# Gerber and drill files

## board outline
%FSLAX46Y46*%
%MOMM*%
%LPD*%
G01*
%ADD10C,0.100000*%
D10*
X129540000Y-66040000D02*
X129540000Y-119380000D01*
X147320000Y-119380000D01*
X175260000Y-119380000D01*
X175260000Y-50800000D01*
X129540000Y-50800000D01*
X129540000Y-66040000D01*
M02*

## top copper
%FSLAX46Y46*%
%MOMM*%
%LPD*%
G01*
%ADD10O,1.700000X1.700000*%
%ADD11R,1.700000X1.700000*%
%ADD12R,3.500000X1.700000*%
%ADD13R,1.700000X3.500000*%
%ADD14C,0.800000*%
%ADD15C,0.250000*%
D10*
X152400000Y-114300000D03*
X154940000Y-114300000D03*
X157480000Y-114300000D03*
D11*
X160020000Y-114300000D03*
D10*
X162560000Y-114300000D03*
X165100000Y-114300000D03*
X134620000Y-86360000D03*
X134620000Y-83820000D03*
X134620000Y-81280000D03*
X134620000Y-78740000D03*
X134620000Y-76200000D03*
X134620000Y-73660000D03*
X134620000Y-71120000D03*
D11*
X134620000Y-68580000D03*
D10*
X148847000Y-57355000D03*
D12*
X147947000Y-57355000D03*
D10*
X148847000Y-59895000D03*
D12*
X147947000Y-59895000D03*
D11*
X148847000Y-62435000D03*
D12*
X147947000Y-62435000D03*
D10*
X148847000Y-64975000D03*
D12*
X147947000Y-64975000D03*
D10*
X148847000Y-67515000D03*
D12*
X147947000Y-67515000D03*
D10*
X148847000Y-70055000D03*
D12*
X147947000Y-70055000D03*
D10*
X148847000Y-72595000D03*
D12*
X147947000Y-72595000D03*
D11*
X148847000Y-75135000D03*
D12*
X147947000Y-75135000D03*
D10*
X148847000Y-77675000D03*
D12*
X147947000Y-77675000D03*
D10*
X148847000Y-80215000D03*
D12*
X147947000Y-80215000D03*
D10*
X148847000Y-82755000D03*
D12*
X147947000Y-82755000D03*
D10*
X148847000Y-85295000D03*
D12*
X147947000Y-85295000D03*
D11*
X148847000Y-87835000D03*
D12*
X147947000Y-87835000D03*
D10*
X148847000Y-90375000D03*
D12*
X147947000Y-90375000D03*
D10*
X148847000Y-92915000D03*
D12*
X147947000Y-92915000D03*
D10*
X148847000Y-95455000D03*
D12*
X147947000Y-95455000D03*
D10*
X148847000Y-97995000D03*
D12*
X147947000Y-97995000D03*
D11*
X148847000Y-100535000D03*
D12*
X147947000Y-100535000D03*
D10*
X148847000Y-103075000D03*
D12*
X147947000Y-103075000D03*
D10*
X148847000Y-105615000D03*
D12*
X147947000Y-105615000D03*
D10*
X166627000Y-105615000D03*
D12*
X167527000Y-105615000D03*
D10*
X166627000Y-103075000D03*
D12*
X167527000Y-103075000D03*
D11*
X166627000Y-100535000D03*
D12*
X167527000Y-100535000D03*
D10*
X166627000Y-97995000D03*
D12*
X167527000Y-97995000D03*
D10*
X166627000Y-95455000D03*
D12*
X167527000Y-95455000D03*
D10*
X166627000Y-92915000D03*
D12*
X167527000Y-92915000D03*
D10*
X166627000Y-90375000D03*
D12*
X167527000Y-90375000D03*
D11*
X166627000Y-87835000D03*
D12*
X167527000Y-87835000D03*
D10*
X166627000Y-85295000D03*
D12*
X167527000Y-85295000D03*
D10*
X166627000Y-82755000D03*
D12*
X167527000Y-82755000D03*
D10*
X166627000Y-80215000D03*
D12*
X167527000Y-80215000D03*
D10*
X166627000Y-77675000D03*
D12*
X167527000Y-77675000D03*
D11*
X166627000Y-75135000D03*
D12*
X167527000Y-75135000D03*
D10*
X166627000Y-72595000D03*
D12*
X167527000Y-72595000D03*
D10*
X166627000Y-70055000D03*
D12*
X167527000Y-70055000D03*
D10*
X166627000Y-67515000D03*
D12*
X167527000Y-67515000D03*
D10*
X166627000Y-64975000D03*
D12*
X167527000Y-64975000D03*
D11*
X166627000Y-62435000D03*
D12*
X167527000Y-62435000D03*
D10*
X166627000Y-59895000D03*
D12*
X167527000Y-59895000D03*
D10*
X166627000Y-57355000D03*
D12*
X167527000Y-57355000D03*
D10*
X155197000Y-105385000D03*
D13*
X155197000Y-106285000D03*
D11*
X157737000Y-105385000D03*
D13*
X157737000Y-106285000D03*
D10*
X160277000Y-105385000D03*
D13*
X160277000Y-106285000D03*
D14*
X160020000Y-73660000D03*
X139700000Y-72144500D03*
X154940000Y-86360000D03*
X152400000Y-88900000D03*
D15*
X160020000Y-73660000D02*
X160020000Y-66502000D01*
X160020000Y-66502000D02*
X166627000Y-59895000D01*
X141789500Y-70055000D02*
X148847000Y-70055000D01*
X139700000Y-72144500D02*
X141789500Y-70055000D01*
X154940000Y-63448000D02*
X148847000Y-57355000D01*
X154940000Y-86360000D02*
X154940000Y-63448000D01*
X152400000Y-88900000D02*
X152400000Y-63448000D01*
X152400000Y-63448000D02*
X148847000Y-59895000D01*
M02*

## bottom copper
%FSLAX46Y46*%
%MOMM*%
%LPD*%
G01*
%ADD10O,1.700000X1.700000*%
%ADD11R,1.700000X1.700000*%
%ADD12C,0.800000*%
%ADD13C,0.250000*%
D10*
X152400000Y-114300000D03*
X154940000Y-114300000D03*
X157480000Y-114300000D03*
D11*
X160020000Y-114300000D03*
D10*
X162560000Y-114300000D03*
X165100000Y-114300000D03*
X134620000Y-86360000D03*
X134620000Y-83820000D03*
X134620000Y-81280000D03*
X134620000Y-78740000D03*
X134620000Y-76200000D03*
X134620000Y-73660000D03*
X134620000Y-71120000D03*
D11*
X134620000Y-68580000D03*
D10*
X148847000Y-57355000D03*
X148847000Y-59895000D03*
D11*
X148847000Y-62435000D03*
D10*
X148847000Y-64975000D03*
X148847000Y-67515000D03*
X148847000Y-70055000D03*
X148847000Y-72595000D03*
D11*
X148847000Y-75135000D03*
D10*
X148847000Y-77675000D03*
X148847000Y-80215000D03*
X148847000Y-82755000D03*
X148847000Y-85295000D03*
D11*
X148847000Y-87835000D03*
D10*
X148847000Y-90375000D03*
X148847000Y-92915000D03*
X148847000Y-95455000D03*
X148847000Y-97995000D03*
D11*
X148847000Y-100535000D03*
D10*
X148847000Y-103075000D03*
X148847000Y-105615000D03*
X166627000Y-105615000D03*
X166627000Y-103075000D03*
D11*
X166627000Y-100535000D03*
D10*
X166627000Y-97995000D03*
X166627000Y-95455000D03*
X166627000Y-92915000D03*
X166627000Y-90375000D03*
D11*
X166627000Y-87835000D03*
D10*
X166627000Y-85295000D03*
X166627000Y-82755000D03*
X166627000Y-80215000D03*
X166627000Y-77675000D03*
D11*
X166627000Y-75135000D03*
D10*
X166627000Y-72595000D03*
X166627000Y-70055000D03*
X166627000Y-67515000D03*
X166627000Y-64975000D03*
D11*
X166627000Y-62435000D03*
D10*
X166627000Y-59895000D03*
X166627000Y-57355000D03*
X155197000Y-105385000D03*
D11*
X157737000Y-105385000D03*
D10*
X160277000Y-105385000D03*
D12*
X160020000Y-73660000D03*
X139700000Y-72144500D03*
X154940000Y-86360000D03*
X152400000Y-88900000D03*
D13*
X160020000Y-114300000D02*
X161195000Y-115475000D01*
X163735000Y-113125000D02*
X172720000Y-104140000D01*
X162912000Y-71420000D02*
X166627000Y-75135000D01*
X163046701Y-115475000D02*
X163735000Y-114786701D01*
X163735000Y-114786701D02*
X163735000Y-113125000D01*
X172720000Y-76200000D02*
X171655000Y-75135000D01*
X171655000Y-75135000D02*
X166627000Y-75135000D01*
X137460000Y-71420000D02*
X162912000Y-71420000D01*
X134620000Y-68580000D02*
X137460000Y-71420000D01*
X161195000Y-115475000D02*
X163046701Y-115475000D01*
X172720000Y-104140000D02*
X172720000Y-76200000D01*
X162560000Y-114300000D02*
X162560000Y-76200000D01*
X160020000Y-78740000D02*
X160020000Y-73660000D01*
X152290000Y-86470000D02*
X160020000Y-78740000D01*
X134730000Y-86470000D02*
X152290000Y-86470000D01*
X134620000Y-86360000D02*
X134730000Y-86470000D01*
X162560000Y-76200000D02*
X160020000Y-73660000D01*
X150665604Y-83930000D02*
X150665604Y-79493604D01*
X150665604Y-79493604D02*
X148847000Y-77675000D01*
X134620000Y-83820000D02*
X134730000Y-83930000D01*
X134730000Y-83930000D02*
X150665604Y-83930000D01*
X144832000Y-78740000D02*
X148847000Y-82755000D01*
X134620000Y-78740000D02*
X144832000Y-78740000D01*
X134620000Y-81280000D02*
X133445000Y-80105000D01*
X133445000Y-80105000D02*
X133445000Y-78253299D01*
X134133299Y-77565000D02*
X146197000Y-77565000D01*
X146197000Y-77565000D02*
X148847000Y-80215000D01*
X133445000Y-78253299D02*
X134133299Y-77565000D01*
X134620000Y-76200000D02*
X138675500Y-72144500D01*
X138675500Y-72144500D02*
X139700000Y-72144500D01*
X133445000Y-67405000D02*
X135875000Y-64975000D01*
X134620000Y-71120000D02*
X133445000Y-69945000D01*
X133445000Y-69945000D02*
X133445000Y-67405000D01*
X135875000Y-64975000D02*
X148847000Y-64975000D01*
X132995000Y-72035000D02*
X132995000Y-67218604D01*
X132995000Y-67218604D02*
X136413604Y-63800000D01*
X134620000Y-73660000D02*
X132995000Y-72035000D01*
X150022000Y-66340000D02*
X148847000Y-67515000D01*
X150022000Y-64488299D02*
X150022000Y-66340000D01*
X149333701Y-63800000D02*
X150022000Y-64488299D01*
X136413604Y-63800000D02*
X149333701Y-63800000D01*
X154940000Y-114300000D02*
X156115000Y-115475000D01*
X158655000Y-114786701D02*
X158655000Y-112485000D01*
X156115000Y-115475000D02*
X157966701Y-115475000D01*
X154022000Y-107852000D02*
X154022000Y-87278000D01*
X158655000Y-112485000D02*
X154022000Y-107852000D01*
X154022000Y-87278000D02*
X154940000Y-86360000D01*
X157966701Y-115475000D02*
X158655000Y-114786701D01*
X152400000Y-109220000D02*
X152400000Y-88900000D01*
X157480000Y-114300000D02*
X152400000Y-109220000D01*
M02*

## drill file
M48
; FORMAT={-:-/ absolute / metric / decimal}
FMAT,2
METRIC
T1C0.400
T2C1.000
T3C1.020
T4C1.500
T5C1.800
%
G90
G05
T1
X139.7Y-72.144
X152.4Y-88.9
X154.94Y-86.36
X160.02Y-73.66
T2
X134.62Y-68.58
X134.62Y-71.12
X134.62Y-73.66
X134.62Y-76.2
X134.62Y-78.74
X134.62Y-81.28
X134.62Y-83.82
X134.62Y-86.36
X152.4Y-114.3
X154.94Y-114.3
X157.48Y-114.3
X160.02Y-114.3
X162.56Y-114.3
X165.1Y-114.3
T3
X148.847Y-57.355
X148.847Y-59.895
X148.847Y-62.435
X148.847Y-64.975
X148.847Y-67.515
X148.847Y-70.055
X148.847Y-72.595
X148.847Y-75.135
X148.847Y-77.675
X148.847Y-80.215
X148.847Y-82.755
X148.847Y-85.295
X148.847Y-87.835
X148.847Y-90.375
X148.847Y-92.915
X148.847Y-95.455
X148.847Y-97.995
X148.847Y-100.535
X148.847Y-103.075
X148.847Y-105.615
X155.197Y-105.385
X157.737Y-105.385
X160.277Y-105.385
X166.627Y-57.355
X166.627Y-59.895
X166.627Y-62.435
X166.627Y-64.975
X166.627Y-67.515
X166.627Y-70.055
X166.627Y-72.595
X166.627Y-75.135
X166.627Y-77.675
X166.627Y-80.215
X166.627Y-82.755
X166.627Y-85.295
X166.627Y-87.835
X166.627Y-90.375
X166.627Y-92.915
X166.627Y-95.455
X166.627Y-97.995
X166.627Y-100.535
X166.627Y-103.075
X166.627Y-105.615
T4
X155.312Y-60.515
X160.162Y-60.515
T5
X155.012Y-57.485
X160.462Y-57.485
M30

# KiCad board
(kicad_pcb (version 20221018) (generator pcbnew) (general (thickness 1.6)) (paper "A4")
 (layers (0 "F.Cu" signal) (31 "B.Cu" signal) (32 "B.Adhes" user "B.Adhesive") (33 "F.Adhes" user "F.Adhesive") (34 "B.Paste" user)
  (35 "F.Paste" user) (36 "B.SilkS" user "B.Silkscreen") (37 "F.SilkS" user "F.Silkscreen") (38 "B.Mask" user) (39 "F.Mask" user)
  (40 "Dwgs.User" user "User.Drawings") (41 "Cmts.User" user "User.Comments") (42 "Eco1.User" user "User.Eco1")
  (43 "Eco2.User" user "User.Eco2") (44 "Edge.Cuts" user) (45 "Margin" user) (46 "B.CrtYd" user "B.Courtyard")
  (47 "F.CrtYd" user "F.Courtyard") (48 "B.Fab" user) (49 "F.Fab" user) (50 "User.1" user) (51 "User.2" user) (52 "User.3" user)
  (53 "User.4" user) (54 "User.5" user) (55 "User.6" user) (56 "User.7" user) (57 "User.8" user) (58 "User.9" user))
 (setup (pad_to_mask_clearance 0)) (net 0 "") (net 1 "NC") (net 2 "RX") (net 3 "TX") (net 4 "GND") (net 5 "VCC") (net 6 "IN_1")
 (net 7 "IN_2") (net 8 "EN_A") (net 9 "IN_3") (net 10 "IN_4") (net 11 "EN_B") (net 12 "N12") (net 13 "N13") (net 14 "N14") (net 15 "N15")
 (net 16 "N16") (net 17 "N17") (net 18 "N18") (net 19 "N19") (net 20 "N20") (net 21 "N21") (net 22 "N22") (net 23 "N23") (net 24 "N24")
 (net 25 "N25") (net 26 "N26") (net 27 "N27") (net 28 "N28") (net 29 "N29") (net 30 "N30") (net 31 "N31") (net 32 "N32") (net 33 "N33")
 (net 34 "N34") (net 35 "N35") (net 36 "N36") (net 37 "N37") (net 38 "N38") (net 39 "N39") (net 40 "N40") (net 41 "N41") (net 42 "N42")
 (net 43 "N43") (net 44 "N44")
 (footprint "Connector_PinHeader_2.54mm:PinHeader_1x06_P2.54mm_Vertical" (layer "F.Cu") (at 152.4 114.3 90)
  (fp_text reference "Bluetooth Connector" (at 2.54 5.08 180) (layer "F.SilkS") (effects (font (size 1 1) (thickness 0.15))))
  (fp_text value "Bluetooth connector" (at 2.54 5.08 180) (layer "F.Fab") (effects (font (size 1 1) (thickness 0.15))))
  (pad "1" thru_hole oval (at 0 0 90) (size 1.7 1.7) (drill 1) (layers "*.Cu" "*.Mask") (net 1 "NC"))
  (pad "2" thru_hole oval (at 0 2.54 90) (size 1.7 1.7) (drill 1) (layers "*.Cu" "*.Mask") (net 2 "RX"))
  (pad "3" thru_hole oval (at 0 5.08 90) (size 1.7 1.7) (drill 1) (layers "*.Cu" "*.Mask") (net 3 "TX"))
  (pad "4" thru_hole rect (at 0 7.62 90) (size 1.7 1.7) (drill 1) (layers "*.Cu" "*.Mask") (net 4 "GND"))
  (pad "5" thru_hole oval (at 0 10.16 90) (size 1.7 1.7) (drill 1) (layers "*.Cu" "*.Mask") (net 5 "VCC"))
  (pad "6" thru_hole oval (at 0 12.7 90) (size 1.7 1.7) (drill 1) (layers "*.Cu" "*.Mask") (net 1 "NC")))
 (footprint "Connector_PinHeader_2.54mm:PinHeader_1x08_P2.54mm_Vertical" (layer "F.Cu") (at 134.62 86.36 180)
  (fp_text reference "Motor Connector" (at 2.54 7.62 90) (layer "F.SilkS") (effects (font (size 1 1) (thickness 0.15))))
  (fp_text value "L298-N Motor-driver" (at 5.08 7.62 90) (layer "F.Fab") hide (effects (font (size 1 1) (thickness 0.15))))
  (pad "1" thru_hole oval (at 0 0 180) (size 1.7 1.7) (drill 1) (layers "*.Cu" "*.Mask") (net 5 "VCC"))
  (pad "2" thru_hole oval (at 0 2.54 180) (size 1.7 1.7) (drill 1) (layers "*.Cu" "*.Mask") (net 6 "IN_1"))
  (pad "3" thru_hole oval (at 0 5.08 180) (size 1.7 1.7) (drill 1) (layers "*.Cu" "*.Mask") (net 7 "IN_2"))
  (pad "4" thru_hole oval (at 0 7.62 180) (size 1.7 1.7) (drill 1) (layers "*.Cu" "*.Mask") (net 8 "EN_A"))
  (pad "5" thru_hole oval (at 0 10.16 180) (size 1.7 1.7) (drill 1) (layers "*.Cu" "*.Mask") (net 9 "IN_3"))
  (pad "6" thru_hole oval (at 0 12.7 180) (size 1.7 1.7) (drill 1) (layers "*.Cu" "*.Mask") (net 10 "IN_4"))
  (pad "7" thru_hole oval (at 0 15.24 180) (size 1.7 1.7) (drill 1) (layers "*.Cu" "*.Mask") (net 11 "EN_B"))
  (pad "8" thru_hole rect (at 0 17.78 180) (size 1.7 1.7) (drill 1) (layers "*.Cu" "*.Mask") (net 4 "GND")))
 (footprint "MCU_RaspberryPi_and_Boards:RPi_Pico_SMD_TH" (layer "F.Cu") (at 157.737 81.485)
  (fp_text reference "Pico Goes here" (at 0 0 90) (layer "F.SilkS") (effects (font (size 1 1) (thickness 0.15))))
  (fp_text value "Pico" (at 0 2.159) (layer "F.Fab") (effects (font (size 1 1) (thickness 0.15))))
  (pad "" np_thru_hole oval (at -2.725 -24) (size 1.8 1.8) (drill 1.8) (layers "*.Cu" "*.Mask"))
  (pad "" np_thru_hole oval (at -2.425 -20.97) (size 1.5 1.5) (drill 1.5) (layers "*.Cu" "*.Mask"))
  (pad "" np_thru_hole oval (at 2.425 -20.97) (size 1.5 1.5) (drill 1.5) (layers "*.Cu" "*.Mask"))
  (pad "" np_thru_hole oval (at 2.725 -24) (size 1.8 1.8) (drill 1.8) (layers "*.Cu" "*.Mask"))
  (pad "1" thru_hole oval (at -8.89 -24.13) (size 1.7 1.7) (drill 1.02) (layers "*.Cu" "*.Mask") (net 2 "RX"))
  (pad "1" smd rect (at -8.89 -24.13) (size 3.5 1.7) (drill (offset -0.9 0)) (layers "F.Cu" "F.Mask") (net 2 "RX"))
  (pad "2" thru_hole oval (at -8.89 -21.59) (size 1.7 1.7) (drill 1.02) (layers "*.Cu" "*.Mask") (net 3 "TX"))
  (pad "2" smd rect (at -8.89 -21.59) (size 3.5 1.7) (drill (offset -0.9 0)) (layers "F.Cu" "F.Mask") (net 3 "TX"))
  (pad "3" thru_hole rect (at -8.89 -19.05) (size 1.7 1.7) (drill 1.02) (layers "*.Cu" "*.Mask") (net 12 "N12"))
  (pad "3" smd rect (at -8.89 -19.05) (size 3.5 1.7) (drill (offset -0.9 0)) (layers "F.Cu" "F.Mask") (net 12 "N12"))
  (pad "4" thru_hole oval (at -8.89 -16.51) (size 1.7 1.7) (drill 1.02) (layers "*.Cu" "*.Mask") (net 11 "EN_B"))
  (pad "4" smd rect (at -8.89 -16.51) (size 3.5 1.7) (drill (offset -0.9 0)) (layers "F.Cu" "F.Mask") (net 11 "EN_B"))
  (pad "5" thru_hole oval (at -8.89 -13.97) (size 1.7 1.7) (drill 1.02) (layers "*.Cu" "*.Mask") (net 10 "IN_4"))
  (pad "5" smd rect (at -8.89 -13.97) (size 3.5 1.7) (drill (offset -0.9 0)) (layers "F.Cu" "F.Mask") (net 10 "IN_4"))
  (pad "6" thru_hole oval (at -8.89 -11.43) (size 1.7 1.7) (drill 1.02) (layers "*.Cu" "*.Mask") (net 9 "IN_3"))
  (pad "6" smd rect (at -8.89 -11.43) (size 3.5 1.7) (drill (offset -0.9 0)) (layers "F.Cu" "F.Mask") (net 9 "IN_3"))
  (pad "7" thru_hole oval (at -8.89 -8.89) (size 1.7 1.7) (drill 1.02) (layers "*.Cu" "*.Mask") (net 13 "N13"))
  (pad "7" smd rect (at -8.89 -8.89) (size 3.5 1.7) (drill (offset -0.9 0)) (layers "F.Cu" "F.Mask") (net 13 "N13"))
  (pad "8" thru_hole rect (at -8.89 -6.35) (size 1.7 1.7) (drill 1.02) (layers "*.Cu" "*.Mask") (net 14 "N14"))
  (pad "8" smd rect (at -8.89 -6.35) (size 3.5 1.7) (drill (offset -0.9 0)) (layers "F.Cu" "F.Mask") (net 14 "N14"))
  (pad "9" thru_hole oval (at -8.89 -3.81) (size 1.7 1.7) (drill 1.02) (layers "*.Cu" "*.Mask") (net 6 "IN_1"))
  (pad "9" smd rect (at -8.89 -3.81) (size 3.5 1.7) (drill (offset -0.9 0)) (layers "F.Cu" "F.Mask") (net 6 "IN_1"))
  (pad "10" thru_hole oval (at -8.89 -1.27) (size 1.7 1.7) (drill 1.02) (layers "*.Cu" "*.Mask") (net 7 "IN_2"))
  (pad "10" smd rect (at -8.89 -1.27) (size 3.5 1.7) (drill (offset -0.9 0)) (layers "F.Cu" "F.Mask") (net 7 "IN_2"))
  (pad "11" thru_hole oval (at -8.89 1.27) (size 1.7 1.7) (drill 1.02) (layers "*.Cu" "*.Mask") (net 8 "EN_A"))
  (pad "11" smd rect (at -8.89 1.27) (size 3.5 1.7) (drill (offset -0.9 0)) (layers "F.Cu" "F.Mask") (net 8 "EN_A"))
  (pad "12" thru_hole oval (at -8.89 3.81) (size 1.7 1.7) (drill 1.02) (layers "*.Cu" "*.Mask") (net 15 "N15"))
  (pad "12" smd rect (at -8.89 3.81) (size 3.5 1.7) (drill (offset -0.9 0)) (layers "F.Cu" "F.Mask") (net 15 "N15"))
  (pad "13" thru_hole rect (at -8.89 6.35) (size 1.7 1.7) (drill 1.02) (layers "*.Cu" "*.Mask") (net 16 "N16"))
  (pad "13" smd rect (at -8.89 6.35) (size 3.5 1.7) (drill (offset -0.9 0)) (layers "F.Cu" "F.Mask") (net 16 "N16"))
  (pad "14" thru_hole oval (at -8.89 8.89) (size 1.7 1.7) (drill 1.02) (layers "*.Cu" "*.Mask") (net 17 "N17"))
  (pad "14" smd rect (at -8.89 8.89) (size 3.5 1.7) (drill (offset -0.9 0)) (layers "F.Cu" "F.Mask") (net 17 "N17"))
  (pad "15" thru_hole oval (at -8.89 11.43) (size 1.7 1.7) (drill 1.02) (layers "*.Cu" "*.Mask") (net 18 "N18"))
  (pad "15" smd rect (at -8.89 11.43) (size 3.5 1.7) (drill (offset -0.9 0)) (layers "F.Cu" "F.Mask") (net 18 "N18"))
  (pad "16" thru_hole oval (at -8.89 13.97) (size 1.7 1.7) (drill 1.02) (layers "*.Cu" "*.Mask") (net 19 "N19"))
  (pad "16" smd rect (at -8.89 13.97) (size 3.5 1.7) (drill (offset -0.9 0)) (layers "F.Cu" "F.Mask") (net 19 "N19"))
  (pad "17" thru_hole oval (at -8.89 16.51) (size 1.7 1.7) (drill 1.02) (layers "*.Cu" "*.Mask") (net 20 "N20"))
  (pad "17" smd rect (at -8.89 16.51) (size 3.5 1.7) (drill (offset -0.9 0)) (layers "F.Cu" "F.Mask") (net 20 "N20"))
  (pad "18" thru_hole rect (at -8.89 19.05) (size 1.7 1.7) (drill 1.02) (layers "*.Cu" "*.Mask") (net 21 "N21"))
  (pad "18" smd rect (at -8.89 19.05) (size 3.5 1.7) (drill (offset -0.9 0)) (layers "F.Cu" "F.Mask") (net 21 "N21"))
  (pad "19" thru_hole oval (at -8.89 21.59) (size 1.7 1.7) (drill 1.02) (layers "*.Cu" "*.Mask") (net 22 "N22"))
  (pad "19" smd rect (at -8.89 21.59) (size 3.5 1.7) (drill (offset -0.9 0)) (layers "F.Cu" "F.Mask") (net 22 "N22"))
  (pad "20" thru_hole oval (at -8.89 24.13) (size 1.7 1.7) (drill 1.02) (layers "*.Cu" "*.Mask") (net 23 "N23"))
  (pad "20" smd rect (at -8.89 24.13) (size 3.5 1.7) (drill (offset -0.9 0)) (layers "F.Cu" "F.Mask") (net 23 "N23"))
  (pad "21" thru_hole oval (at 8.89 24.13) (size 1.7 1.7) (drill 1.02) (layers "*.Cu" "*.Mask") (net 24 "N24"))
  (pad "21" smd rect (at 8.89 24.13) (size 3.5 1.7) (drill (offset 0.9 0)) (layers "F.Cu" "F.Mask") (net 24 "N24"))
  (pad "22" thru_hole oval (at 8.89 21.59) (size 1.7 1.7) (drill 1.02) (layers "*.Cu" "*.Mask") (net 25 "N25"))
  (pad "22" smd rect (at 8.89 21.59) (size 3.5 1.7) (drill (offset 0.9 0)) (layers "F.Cu" "F.Mask") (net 25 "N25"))
  (pad "23" thru_hole rect (at 8.89 19.05) (size 1.7 1.7) (drill 1.02) (layers "*.Cu" "*.Mask") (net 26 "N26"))
  (pad "23" smd rect (at 8.89 19.05) (size 3.5 1.7) (drill (offset 0.9 0)) (layers "F.Cu" "F.Mask") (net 26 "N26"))
  (pad "24" thru_hole oval (at 8.89 16.51) (size 1.7 1.7) (drill 1.02) (layers "*.Cu" "*.Mask") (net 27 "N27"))
  (pad "24" smd rect (at 8.89 16.51) (size 3.5 1.7) (drill (offset 0.9 0)) (layers "F.Cu" "F.Mask") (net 27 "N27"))
  (pad "25" thru_hole oval (at 8.89 13.97) (size 1.7 1.7) (drill 1.02) (layers "*.Cu" "*.Mask") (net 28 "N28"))
  (pad "25" smd rect (at 8.89 13.97) (size 3.5 1.7) (drill (offset 0.9 0)) (layers "F.Cu" "F.Mask") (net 28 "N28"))
  (pad "26" thru_hole oval (at 8.89 11.43) (size 1.7 1.7) (drill 1.02) (layers "*.Cu" "*.Mask") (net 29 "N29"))
  (pad "26" smd rect (at 8.89 11.43) (size 3.5 1.7) (drill (offset 0.9 0)) (layers "F.Cu" "F.Mask") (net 29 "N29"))
  (pad "27" thru_hole oval (at 8.89 8.89) (size 1.7 1.7) (drill 1.02) (layers "*.Cu" "*.Mask") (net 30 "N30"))
  (pad "27" smd rect (at 8.89 8.89) (size 3.5 1.7) (drill (offset 0.9 0)) (layers "F.Cu" "F.Mask") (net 30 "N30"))
  (pad "28" thru_hole rect (at 8.89 6.35) (size 1.7 1.7) (drill 1.02) (layers "*.Cu" "*.Mask") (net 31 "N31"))
  (pad "28" smd rect (at 8.89 6.35) (size 3.5 1.7) (drill (offset 0.9 0)) (layers "F.Cu" "F.Mask") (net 31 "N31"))
  (pad "29" thru_hole oval (at 8.89 3.81) (size 1.7 1.7) (drill 1.02) (layers "*.Cu" "*.Mask") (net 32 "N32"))
  (pad "29" smd rect (at 8.89 3.81) (size 3.5 1.7) (drill (offset 0.9 0)) (layers "F.Cu" "F.Mask") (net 32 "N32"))
  (pad "30" thru_hole oval (at 8.89 1.27) (size 1.7 1.7) (drill 1.02) (layers "*.Cu" "*.Mask") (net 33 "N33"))
  (pad "30" smd rect (at 8.89 1.27) (size 3.5 1.7) (drill (offset 0.9 0)) (layers "F.Cu" "F.Mask") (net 33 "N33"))
  (pad "31" thru_hole oval (at 8.89 -1.27) (size 1.7 1.7) (drill 1.02) (layers "*.Cu" "*.Mask") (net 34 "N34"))
  (pad "31" smd rect (at 8.89 -1.27) (size 3.5 1.7) (drill (offset 0.9 0)) (layers "F.Cu" "F.Mask") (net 34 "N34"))
  (pad "32" thru_hole oval (at 8.89 -3.81) (size 1.7 1.7) (drill 1.02) (layers "*.Cu" "*.Mask") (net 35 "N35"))
  (pad "32" smd rect (at 8.89 -3.81) (size 3.5 1.7) (drill (offset 0.9 0)) (layers "F.Cu" "F.Mask") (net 35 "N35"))
  (pad "33" thru_hole rect (at 8.89 -6.35) (size 1.7 1.7) (drill 1.02) (layers "*.Cu" "*.Mask") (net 4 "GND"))
  (pad "33" smd rect (at 8.89 -6.35) (size 3.5 1.7) (drill (offset 0.9 0)) (layers "F.Cu" "F.Mask") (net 4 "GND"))
  (pad "34" thru_hole oval (at 8.89 -8.89) (size 1.7 1.7) (drill 1.02) (layers "*.Cu" "*.Mask") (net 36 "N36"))
  (pad "34" smd rect (at 8.89 -8.89) (size 3.5 1.7) (drill (offset 0.9 0)) (layers "F.Cu" "F.Mask") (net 36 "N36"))
  (pad "35" thru_hole oval (at 8.89 -11.43) (size 1.7 1.7) (drill 1.02) (layers "*.Cu" "*.Mask") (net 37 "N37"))
  (pad "35" smd rect (at 8.89 -11.43) (size 3.5 1.7) (drill (offset 0.9 0)) (layers "F.Cu" "F.Mask") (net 37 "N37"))
  (pad "36" thru_hole oval (at 8.89 -13.97) (size 1.7 1.7) (drill 1.02) (layers "*.Cu" "*.Mask") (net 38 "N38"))
  (pad "36" smd rect (at 8.89 -13.97) (size 3.5 1.7) (drill (offset 0.9 0)) (layers "F.Cu" "F.Mask") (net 38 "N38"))
  (pad "37" thru_hole oval (at 8.89 -16.51) (size 1.7 1.7) (drill 1.02) (layers "*.Cu" "*.Mask") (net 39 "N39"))
  (pad "37" smd rect (at 8.89 -16.51) (size 3.5 1.7) (drill (offset 0.9 0)) (layers "F.Cu" "F.Mask") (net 39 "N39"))
  (pad "38" thru_hole rect (at 8.89 -19.05) (size 1.7 1.7) (drill 1.02) (layers "*.Cu" "*.Mask") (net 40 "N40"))
  (pad "38" smd rect (at 8.89 -19.05) (size 3.5 1.7) (drill (offset 0.9 0)) (layers "F.Cu" "F.Mask") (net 40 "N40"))
  (pad "39" thru_hole oval (at 8.89 -21.59) (size 1.7 1.7) (drill 1.02) (layers "*.Cu" "*.Mask") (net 5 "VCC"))
  (pad "39" smd rect (at 8.89 -21.59) (size 3.5 1.7) (drill (offset 0.9 0)) (layers "F.Cu" "F.Mask") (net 5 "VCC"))
  (pad "40" thru_hole oval (at 8.89 -24.13) (size 1.7 1.7) (drill 1.02) (layers "*.Cu" "*.Mask") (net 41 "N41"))
  (pad "40" smd rect (at 8.89 -24.13) (size 3.5 1.7) (drill (offset 0.9 0)) (layers "F.Cu" "F.Mask") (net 41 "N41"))
  (pad "41" thru_hole oval (at -2.54 23.9) (size 1.7 1.7) (drill 1.02) (layers "*.Cu" "*.Mask") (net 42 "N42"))
  (pad "41" smd rect (at -2.54 23.9 90) (size 3.5 1.7) (drill (offset -0.9 0)) (layers "F.Cu" "F.Mask") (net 42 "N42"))
  (pad "42" thru_hole rect (at 0 23.9) (size 1.7 1.7) (drill 1.02) (layers "*.Cu" "*.Mask") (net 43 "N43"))
  (pad "42" smd rect (at 0 23.9 90) (size 3.5 1.7) (drill (offset -0.9 0)) (layers "F.Cu" "F.Mask") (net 43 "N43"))
  (pad "43" thru_hole oval (at 2.54 23.9) (size 1.7 1.7) (drill 1.02) (layers "*.Cu" "*.Mask") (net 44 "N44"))
  (pad "43" smd rect (at 2.54 23.9 90) (size 3.5 1.7) (drill (offset -0.9 0)) (layers "F.Cu" "F.Mask") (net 44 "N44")))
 (gr_poly
  (pts (xy 129.54 66.04) (xy 129.54 119.38) (xy 147.32 119.38) (xy 175.26 119.38) (xy 175.26 50.8) (xy 129.54 50.8))
  (stroke (width 0.1) (type solid)) (fill none) (layer "Edge.Cuts"))
 (segment (start 160.02 114.3) (end 161.195 115.475) (width 0.25) (layer "B.Cu") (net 4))
 (segment (start 163.735 113.125) (end 172.72 104.14) (width 0.25) (layer "B.Cu") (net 4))
 (segment (start 162.912 71.42) (end 166.627 75.135) (width 0.25) (layer "B.Cu") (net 4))
 (segment (start 163.046701 115.475) (end 163.735 114.786701) (width 0.25) (layer "B.Cu") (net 4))
 (segment (start 163.735 114.786701) (end 163.735 113.125) (width 0.25) (layer "B.Cu") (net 4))
 (segment (start 172.72 76.2) (end 171.655 75.135) (width 0.25) (layer "B.Cu") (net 4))
 (segment (start 171.655 75.135) (end 166.627 75.135) (width 0.25) (layer "B.Cu") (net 4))
 (segment (start 137.46 71.42) (end 162.912 71.42) (width 0.25) (layer "B.Cu") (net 4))
 (segment (start 134.62 68.58) (end 137.46 71.42) (width 0.25) (layer "B.Cu") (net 4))
 (segment (start 161.195 115.475) (end 163.046701 115.475) (width 0.25) (layer "B.Cu") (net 4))
 (segment (start 172.72 104.14) (end 172.72 76.2) (width 0.25) (layer "B.Cu") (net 4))
 (segment (start 160.02 73.66) (end 160.02 66.502) (width 0.25) (layer "F.Cu") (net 5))
 (segment (start 160.02 66.502) (end 166.627 59.895) (width 0.25) (layer "F.Cu") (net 5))
 (via (at 160.02 73.66) (size 0.8) (drill 0.4) (layers "F.Cu" "B.Cu") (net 5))
 (segment (start 162.56 114.3) (end 162.56 76.2) (width 0.25) (layer "B.Cu") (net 5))
 (segment (start 160.02 78.74) (end 160.02 73.66) (width 0.25) (layer "B.Cu") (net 5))
 (segment (start 152.29 86.47) (end 160.02 78.74) (width 0.25) (layer "B.Cu") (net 5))
 (segment (start 134.73 86.47) (end 152.29 86.47) (width 0.25) (layer "B.Cu") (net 5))
 (segment (start 134.62 86.36) (end 134.73 86.47) (width 0.25) (layer "B.Cu") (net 5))
 (segment (start 162.56 76.2) (end 160.02 73.66) (width 0.25) (layer "B.Cu") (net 5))
 (segment (start 150.665604 83.93) (end 150.665604 79.493604) (width 0.25) (layer "B.Cu") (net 6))
 (segment (start 150.665604 79.493604) (end 148.847 77.675) (width 0.25) (layer "B.Cu") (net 6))
 (segment (start 134.62 83.82) (end 134.73 83.93) (width 0.25) (layer "B.Cu") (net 6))
 (segment (start 134.73 83.93) (end 150.665604 83.93) (width 0.25) (layer "B.Cu") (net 6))
 (segment (start 144.832 78.74) (end 148.847 82.755) (width 0.25) (layer "B.Cu") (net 8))
 (segment (start 134.62 78.74) (end 144.832 78.74) (width 0.25) (layer "B.Cu") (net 8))
 (segment (start 134.62 81.28) (end 133.445 80.105) (width 0.25) (layer "B.Cu") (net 7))
 (segment (start 133.445 80.105) (end 133.445 78.253299) (width 0.25) (layer "B.Cu") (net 7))
 (segment (start 134.133299 77.565) (end 146.197 77.565) (width 0.25) (layer "B.Cu") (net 7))
 (segment (start 146.197 77.565) (end 148.847 80.215) (width 0.25) (layer "B.Cu") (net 7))
 (segment (start 133.445 78.253299) (end 134.133299 77.565) (width 0.25) (layer "B.Cu") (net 7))
 (segment (start 141.7895 70.055) (end 148.847 70.055) (width 0.25) (layer "F.Cu") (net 9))
 (segment (start 139.7 72.1445) (end 141.7895 70.055) (width 0.25) (layer "F.Cu") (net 9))
 (via (at 139.7 72.1445) (size 0.8) (drill 0.4) (layers "F.Cu" "B.Cu") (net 9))
 (segment (start 134.62 76.2) (end 138.6755 72.1445) (width 0.25) (layer "B.Cu") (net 9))
 (segment (start 138.6755 72.1445) (end 139.7 72.1445) (width 0.25) (layer "B.Cu") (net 9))
 (segment (start 133.445 67.405) (end 135.875 64.975) (width 0.25) (layer "B.Cu") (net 11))
 (segment (start 134.62 71.12) (end 133.445 69.945) (width 0.25) (layer "B.Cu") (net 11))
 (segment (start 133.445 69.945) (end 133.445 67.405) (width 0.25) (layer "B.Cu") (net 11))
 (segment (start 135.875 64.975) (end 148.847 64.975) (width 0.25) (layer "B.Cu") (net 11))
 (segment (start 132.995 72.035) (end 132.995 67.218604) (width 0.25) (layer "B.Cu") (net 10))
 (segment (start 132.995 67.218604) (end 136.413604 63.8) (width 0.25) (layer "B.Cu") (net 10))
 (segment (start 134.62 73.66) (end 132.995 72.035) (width 0.25) (layer "B.Cu") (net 10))
 (segment (start 150.022 66.34) (end 148.847 67.515) (width 0.25) (layer "B.Cu") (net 10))
 (segment (start 150.022 64.488299) (end 150.022 66.34) (width 0.25) (layer "B.Cu") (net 10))
 (segment (start 149.333701 63.8) (end 150.022 64.488299) (width 0.25) (layer "B.Cu") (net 10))
 (segment (start 136.413604 63.8) (end 149.333701 63.8) (width 0.25) (layer "B.Cu") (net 10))
 (segment (start 154.94 63.448) (end 148.847 57.355) (width 0.25) (layer "F.Cu") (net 2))
 (segment (start 154.94 86.36) (end 154.94 63.448) (width 0.25) (layer "F.Cu") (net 2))
 (via (at 154.94 86.36) (size 0.8) (drill 0.4) (layers "F.Cu" "B.Cu") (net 2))
 (segment (start 154.94 114.3) (end 156.115 115.475) (width 0.25) (layer "B.Cu") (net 2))
 (segment (start 158.655 114.786701) (end 158.655 112.485) (width 0.25) (layer "B.Cu") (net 2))
 (segment (start 156.115 115.475) (end 157.966701 115.475) (width 0.25) (layer "B.Cu") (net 2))
 (segment (start 154.022 107.852) (end 154.022 87.278) (width 0.25) (layer "B.Cu") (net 2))
 (segment (start 158.655 112.485) (end 154.022 107.852) (width 0.25) (layer "B.Cu") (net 2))
 (segment (start 154.022 87.278) (end 154.94 86.36) (width 0.25) (layer "B.Cu") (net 2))
 (segment (start 157.966701 115.475) (end 158.655 114.786701) (width 0.25) (layer "B.Cu") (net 2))
 (segment (start 152.4 88.9) (end 152.4 63.448) (width 0.25) (layer "F.Cu") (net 3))
 (segment (start 152.4 63.448) (end 148.847 59.895) (width 0.25) (layer "F.Cu") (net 3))
 (via (at 152.4 88.9) (size 0.8) (drill 0.4) (layers "F.Cu" "B.Cu") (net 3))
 (segment (start 152.4 109.22) (end 152.4 88.9) (width 0.25) (layer "B.Cu") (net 3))
 (segment (start 157.48 114.3) (end 152.4 109.22) (width 0.25) (layer "B.Cu") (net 3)))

